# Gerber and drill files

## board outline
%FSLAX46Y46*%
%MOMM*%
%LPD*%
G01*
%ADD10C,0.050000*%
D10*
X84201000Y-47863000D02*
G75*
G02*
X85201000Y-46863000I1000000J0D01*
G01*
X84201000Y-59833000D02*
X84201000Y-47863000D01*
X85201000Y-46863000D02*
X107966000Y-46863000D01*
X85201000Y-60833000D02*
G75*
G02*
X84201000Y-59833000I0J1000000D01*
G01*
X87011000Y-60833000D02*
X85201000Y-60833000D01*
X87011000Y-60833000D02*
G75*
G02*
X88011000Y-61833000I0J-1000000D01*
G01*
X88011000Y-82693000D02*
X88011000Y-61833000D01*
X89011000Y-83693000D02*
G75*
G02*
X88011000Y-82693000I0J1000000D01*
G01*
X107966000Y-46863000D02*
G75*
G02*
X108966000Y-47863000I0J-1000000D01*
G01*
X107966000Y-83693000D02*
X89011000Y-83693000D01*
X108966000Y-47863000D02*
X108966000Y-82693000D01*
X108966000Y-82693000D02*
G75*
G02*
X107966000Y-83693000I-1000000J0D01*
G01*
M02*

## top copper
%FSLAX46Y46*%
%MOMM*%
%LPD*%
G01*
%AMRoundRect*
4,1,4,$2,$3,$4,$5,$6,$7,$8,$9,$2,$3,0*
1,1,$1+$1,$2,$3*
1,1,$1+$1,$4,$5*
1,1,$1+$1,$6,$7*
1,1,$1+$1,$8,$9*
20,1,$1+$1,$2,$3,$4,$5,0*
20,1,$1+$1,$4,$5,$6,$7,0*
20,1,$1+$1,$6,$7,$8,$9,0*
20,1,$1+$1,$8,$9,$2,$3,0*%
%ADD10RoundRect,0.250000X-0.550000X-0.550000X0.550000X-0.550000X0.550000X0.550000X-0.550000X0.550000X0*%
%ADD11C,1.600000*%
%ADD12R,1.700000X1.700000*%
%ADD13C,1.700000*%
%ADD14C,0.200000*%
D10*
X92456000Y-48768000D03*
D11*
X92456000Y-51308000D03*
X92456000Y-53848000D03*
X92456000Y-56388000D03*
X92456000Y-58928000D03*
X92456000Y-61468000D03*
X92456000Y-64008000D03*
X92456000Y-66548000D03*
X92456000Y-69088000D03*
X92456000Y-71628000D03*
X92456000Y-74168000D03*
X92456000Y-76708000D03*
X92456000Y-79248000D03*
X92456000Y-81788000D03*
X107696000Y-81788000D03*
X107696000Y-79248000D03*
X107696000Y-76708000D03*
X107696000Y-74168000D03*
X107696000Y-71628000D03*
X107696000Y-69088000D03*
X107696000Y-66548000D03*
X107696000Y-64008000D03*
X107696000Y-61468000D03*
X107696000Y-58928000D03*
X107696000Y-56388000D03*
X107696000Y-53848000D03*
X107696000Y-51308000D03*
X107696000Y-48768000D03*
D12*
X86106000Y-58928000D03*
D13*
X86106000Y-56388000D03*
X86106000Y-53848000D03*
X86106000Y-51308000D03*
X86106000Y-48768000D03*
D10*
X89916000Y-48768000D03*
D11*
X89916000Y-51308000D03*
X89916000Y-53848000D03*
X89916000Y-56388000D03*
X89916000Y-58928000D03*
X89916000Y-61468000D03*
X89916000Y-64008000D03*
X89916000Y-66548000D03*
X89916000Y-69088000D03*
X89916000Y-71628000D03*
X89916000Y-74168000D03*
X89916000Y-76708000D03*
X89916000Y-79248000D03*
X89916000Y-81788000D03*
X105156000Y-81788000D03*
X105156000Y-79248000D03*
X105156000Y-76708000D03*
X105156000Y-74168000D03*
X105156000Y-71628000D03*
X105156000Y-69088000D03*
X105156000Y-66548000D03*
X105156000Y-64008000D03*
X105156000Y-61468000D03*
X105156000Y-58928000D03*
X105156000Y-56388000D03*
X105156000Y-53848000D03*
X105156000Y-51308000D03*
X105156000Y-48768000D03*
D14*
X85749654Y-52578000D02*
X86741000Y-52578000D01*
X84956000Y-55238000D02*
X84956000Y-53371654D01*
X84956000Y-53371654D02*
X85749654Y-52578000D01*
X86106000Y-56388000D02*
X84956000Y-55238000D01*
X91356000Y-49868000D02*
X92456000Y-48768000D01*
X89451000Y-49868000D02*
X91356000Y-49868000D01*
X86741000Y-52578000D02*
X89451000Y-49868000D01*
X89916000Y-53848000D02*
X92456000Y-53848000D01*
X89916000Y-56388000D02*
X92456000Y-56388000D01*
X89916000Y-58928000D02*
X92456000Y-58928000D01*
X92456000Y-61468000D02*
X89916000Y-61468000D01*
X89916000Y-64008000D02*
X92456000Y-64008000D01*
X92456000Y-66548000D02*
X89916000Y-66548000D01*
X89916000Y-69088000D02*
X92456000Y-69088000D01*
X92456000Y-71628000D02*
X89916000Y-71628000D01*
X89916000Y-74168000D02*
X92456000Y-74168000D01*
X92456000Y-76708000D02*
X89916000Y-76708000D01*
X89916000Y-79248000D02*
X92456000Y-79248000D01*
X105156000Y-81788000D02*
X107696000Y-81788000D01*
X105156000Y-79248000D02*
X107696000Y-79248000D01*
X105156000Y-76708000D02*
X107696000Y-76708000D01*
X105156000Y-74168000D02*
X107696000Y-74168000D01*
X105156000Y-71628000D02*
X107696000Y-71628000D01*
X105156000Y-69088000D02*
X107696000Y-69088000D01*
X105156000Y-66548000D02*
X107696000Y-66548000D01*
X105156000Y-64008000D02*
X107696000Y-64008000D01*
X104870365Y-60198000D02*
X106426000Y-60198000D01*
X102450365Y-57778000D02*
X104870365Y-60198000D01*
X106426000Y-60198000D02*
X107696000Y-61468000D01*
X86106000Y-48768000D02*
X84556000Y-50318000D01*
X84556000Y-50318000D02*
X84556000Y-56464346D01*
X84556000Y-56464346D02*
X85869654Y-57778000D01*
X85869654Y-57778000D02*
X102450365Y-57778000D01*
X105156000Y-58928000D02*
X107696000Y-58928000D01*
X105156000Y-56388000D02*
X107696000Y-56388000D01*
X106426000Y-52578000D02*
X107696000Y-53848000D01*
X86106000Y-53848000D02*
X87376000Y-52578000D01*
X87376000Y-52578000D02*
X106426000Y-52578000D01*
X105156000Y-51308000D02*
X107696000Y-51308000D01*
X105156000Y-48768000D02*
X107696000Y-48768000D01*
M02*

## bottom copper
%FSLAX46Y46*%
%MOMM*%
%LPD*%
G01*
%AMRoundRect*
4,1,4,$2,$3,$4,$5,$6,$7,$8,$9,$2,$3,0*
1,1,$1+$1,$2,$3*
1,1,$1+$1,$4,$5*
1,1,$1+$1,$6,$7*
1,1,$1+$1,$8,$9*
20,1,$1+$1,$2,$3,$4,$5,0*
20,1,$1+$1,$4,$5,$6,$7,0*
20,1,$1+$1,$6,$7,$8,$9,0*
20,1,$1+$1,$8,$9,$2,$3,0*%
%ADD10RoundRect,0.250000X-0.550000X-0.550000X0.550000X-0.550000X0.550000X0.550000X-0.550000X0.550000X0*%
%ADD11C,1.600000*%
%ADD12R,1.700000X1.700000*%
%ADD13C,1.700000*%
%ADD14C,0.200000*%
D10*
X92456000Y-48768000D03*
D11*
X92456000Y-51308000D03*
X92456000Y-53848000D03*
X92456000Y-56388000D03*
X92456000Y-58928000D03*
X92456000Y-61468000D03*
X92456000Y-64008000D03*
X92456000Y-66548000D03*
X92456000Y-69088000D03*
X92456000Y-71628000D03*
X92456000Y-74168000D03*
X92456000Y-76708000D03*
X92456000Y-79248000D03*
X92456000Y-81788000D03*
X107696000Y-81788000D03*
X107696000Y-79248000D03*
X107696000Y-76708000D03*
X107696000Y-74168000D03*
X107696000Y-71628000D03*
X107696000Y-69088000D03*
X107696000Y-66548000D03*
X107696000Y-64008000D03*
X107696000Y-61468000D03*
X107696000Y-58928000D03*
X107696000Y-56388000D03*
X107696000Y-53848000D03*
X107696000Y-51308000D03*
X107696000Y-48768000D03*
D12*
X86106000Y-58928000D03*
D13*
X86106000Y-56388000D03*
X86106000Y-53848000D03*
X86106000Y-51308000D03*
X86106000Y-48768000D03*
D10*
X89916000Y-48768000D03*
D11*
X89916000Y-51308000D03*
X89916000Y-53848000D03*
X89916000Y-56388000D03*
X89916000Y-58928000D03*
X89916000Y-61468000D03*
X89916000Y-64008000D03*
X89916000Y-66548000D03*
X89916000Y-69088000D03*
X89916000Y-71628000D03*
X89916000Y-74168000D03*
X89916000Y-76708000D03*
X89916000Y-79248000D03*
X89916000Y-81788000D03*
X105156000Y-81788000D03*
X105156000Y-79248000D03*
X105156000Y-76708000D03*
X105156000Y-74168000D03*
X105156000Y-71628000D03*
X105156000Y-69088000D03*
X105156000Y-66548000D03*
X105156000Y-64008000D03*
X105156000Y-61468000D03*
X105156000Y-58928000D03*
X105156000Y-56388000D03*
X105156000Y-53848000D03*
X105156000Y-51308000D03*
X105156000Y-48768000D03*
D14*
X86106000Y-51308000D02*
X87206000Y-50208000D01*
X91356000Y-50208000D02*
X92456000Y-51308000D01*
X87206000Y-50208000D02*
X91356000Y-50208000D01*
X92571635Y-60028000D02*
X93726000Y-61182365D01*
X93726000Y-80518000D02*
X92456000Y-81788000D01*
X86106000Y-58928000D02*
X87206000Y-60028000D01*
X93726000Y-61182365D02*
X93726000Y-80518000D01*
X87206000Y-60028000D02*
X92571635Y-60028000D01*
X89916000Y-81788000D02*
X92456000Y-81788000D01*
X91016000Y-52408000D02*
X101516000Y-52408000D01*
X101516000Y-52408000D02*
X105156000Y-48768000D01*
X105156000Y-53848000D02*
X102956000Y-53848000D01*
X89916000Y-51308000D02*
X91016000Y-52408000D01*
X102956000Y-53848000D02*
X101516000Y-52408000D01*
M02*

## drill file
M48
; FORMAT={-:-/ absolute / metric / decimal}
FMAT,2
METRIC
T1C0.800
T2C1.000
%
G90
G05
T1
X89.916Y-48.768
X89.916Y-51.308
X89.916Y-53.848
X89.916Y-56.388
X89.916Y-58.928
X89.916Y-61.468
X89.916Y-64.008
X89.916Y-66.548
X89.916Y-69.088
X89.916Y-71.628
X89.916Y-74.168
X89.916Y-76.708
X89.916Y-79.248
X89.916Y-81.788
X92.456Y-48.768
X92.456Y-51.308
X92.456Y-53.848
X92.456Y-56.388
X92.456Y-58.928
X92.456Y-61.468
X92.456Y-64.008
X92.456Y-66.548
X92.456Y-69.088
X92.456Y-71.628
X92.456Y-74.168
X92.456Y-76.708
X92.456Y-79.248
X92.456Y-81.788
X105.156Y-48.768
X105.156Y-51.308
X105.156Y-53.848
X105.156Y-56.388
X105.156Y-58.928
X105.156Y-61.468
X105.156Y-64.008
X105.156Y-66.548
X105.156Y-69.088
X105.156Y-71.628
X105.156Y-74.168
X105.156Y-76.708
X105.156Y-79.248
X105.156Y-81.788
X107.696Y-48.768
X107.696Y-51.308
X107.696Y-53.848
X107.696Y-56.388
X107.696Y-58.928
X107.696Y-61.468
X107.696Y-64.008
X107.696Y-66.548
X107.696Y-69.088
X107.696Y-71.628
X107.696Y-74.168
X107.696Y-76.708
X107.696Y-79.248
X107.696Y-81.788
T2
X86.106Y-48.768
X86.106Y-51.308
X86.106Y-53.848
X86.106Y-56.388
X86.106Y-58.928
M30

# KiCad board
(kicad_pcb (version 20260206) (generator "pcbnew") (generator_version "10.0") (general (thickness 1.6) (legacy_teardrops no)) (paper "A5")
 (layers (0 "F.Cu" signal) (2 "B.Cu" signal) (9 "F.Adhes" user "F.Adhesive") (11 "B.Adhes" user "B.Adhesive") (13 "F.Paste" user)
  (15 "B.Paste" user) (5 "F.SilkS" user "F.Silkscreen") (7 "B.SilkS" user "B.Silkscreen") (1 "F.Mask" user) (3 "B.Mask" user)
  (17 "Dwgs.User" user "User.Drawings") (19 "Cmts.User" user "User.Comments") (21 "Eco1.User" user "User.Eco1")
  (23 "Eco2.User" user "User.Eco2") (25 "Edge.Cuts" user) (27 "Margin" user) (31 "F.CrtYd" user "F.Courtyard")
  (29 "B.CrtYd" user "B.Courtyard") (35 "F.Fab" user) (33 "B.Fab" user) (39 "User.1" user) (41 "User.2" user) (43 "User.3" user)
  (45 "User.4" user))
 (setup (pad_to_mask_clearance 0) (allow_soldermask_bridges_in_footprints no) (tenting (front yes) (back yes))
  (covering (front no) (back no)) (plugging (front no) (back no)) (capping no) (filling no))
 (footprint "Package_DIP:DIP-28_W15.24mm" (layer "F.Cu") (at 92.456 48.768)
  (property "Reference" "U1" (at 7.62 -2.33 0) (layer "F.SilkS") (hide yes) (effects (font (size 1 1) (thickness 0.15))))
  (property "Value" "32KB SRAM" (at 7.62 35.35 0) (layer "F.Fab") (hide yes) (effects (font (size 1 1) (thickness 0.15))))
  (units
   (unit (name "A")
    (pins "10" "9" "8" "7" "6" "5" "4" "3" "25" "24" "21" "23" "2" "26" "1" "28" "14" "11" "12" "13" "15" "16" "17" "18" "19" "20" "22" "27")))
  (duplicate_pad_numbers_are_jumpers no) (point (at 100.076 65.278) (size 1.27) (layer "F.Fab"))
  (pad "1" thru_hole roundrect (at 0 0) (size 1.6 1.6) (drill 0.8) (layers "*.Cu" "*.Mask") (remove_unused_layers no)
   (roundrect_rratio 0.15625) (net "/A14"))
  (pad "2" thru_hole circle (at 0 2.54) (size 1.6 1.6) (drill 0.8) (layers "*.Cu" "*.Mask") (remove_unused_layers no) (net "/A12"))
  (pad "3" thru_hole circle (at 0 5.08) (size 1.6 1.6) (drill 0.8) (layers "*.Cu" "*.Mask") (remove_unused_layers no) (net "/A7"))
  (pad "4" thru_hole circle (at 0 7.62) (size 1.6 1.6) (drill 0.8) (layers "*.Cu" "*.Mask") (remove_unused_layers no) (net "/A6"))
  (pad "5" thru_hole circle (at 0 10.16) (size 1.6 1.6) (drill 0.8) (layers "*.Cu" "*.Mask") (remove_unused_layers no) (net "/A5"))
  (pad "6" thru_hole circle (at 0 12.7) (size 1.6 1.6) (drill 0.8) (layers "*.Cu" "*.Mask") (remove_unused_layers no) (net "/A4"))
  (pad "7" thru_hole circle (at 0 15.24) (size 1.6 1.6) (drill 0.8) (layers "*.Cu" "*.Mask") (remove_unused_layers no) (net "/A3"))
  (pad "8" thru_hole circle (at 0 17.78) (size 1.6 1.6) (drill 0.8) (layers "*.Cu" "*.Mask") (remove_unused_layers no) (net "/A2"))
  (pad "9" thru_hole circle (at 0 20.32) (size 1.6 1.6) (drill 0.8) (layers "*.Cu" "*.Mask") (remove_unused_layers no) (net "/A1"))
  (pad "10" thru_hole circle (at 0 22.86) (size 1.6 1.6) (drill 0.8) (layers "*.Cu" "*.Mask") (remove_unused_layers no) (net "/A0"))
  (pad "11" thru_hole circle (at 0 25.4) (size 1.6 1.6) (drill 0.8) (layers "*.Cu" "*.Mask") (remove_unused_layers no) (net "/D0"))
  (pad "12" thru_hole circle (at 0 27.94) (size 1.6 1.6) (drill 0.8) (layers "*.Cu" "*.Mask") (remove_unused_layers no) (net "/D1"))
  (pad "13" thru_hole circle (at 0 30.48) (size 1.6 1.6) (drill 0.8) (layers "*.Cu" "*.Mask") (remove_unused_layers no) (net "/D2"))
  (pad "14" thru_hole circle (at 0 33.02) (size 1.6 1.6) (drill 0.8) (layers "*.Cu" "*.Mask") (remove_unused_layers no) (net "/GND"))
  (pad "15" thru_hole circle (at 15.24 33.02) (size 1.6 1.6) (drill 0.8) (layers "*.Cu" "*.Mask") (remove_unused_layers no) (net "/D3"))
  (pad "16" thru_hole circle (at 15.24 30.48) (size 1.6 1.6) (drill 0.8) (layers "*.Cu" "*.Mask") (remove_unused_layers no) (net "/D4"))
  (pad "17" thru_hole circle (at 15.24 27.94) (size 1.6 1.6) (drill 0.8) (layers "*.Cu" "*.Mask") (remove_unused_layers no) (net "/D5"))
  (pad "18" thru_hole circle (at 15.24 25.4) (size 1.6 1.6) (drill 0.8) (layers "*.Cu" "*.Mask") (remove_unused_layers no) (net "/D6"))
  (pad "19" thru_hole circle (at 15.24 22.86) (size 1.6 1.6) (drill 0.8) (layers "*.Cu" "*.Mask") (remove_unused_layers no) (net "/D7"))
  (pad "20" thru_hole circle (at 15.24 20.32) (size 1.6 1.6) (drill 0.8) (layers "*.Cu" "*.Mask") (remove_unused_layers no) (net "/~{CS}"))
  (pad "21" thru_hole circle (at 15.24 17.78) (size 1.6 1.6) (drill 0.8) (layers "*.Cu" "*.Mask") (remove_unused_layers no) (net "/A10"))
  (pad "22" thru_hole circle (at 15.24 15.24) (size 1.6 1.6) (drill 0.8) (layers "*.Cu" "*.Mask") (remove_unused_layers no) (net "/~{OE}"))
  (pad "23" thru_hole circle (at 15.24 12.7) (size 1.6 1.6) (drill 0.8) (layers "*.Cu" "*.Mask") (remove_unused_layers no) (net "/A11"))
  (pad "24" thru_hole circle (at 15.24 10.16) (size 1.6 1.6) (drill 0.8) (layers "*.Cu" "*.Mask") (remove_unused_layers no) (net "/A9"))
  (pad "25" thru_hole circle (at 15.24 7.62) (size 1.6 1.6) (drill 0.8) (layers "*.Cu" "*.Mask") (remove_unused_layers no) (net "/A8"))
  (pad "26" thru_hole circle (at 15.24 5.08) (size 1.6 1.6) (drill 0.8) (layers "*.Cu" "*.Mask") (remove_unused_layers no) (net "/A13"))
  (pad "27" thru_hole circle (at 15.24 2.54) (size 1.6 1.6) (drill 0.8) (layers "*.Cu" "*.Mask") (remove_unused_layers no) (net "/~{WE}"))
  (pad "28" thru_hole circle (at 15.24 0) (size 1.6 1.6) (drill 0.8) (layers "*.Cu" "*.Mask") (remove_unused_layers no) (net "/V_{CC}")))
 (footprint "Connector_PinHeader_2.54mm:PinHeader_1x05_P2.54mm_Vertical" (layer "F.Cu") (at 86.106 58.928 180)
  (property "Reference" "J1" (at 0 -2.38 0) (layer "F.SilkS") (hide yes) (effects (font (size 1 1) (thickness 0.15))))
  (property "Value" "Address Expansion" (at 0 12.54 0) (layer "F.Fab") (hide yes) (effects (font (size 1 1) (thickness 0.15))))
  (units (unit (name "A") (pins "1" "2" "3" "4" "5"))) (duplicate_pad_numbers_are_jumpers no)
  (pad "1" thru_hole rect (at 0 0 180) (size 1.7 1.7) (drill 1) (layers "*.Cu" "*.Mask") (remove_unused_layers no) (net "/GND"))
  (pad "2" thru_hole circle (at 0 2.54 180) (size 1.7 1.7) (drill 1) (layers "*.Cu" "*.Mask") (remove_unused_layers no) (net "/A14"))
  (pad "3" thru_hole circle (at 0 5.08 180) (size 1.7 1.7) (drill 1) (layers "*.Cu" "*.Mask") (remove_unused_layers no) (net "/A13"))
  (pad "4" thru_hole circle (at 0 7.62 180) (size 1.7 1.7) (drill 1) (layers "*.Cu" "*.Mask") (remove_unused_layers no) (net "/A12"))
  (pad "5" thru_hole circle (at 0 10.16 180) (size 1.7 1.7) (drill 1) (layers "*.Cu" "*.Mask") (remove_unused_layers no) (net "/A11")))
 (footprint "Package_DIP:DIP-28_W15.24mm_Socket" (layer "F.Cu") (at 89.916 48.768)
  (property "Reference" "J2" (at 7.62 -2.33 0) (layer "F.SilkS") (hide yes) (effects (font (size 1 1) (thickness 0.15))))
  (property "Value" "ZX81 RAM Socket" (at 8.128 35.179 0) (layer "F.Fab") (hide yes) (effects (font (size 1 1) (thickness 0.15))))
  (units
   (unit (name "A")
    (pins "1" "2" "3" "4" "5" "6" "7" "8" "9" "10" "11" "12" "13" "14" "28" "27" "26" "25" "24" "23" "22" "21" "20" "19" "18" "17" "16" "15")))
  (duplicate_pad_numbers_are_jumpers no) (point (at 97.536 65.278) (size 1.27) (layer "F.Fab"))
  (pad "1" thru_hole roundrect (at 0 0) (size 1.6 1.6) (drill 0.8) (layers "*.Cu" "*.Mask") (remove_unused_layers no)
   (roundrect_rratio 0.15625) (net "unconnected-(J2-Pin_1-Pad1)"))
  (pad "2" thru_hole circle (at 0 2.54) (size 1.6 1.6) (drill 0.8) (layers "*.Cu" "*.Mask") (remove_unused_layers no) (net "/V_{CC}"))
  (pad "3" thru_hole circle (at 0 5.08) (size 1.6 1.6) (drill 0.8) (layers "*.Cu" "*.Mask") (remove_unused_layers no) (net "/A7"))
  (pad "4" thru_hole circle (at 0 7.62) (size 1.6 1.6) (drill 0.8) (layers "*.Cu" "*.Mask") (remove_unused_layers no) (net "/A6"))
  (pad "5" thru_hole circle (at 0 10.16) (size 1.6 1.6) (drill 0.8) (layers "*.Cu" "*.Mask") (remove_unused_layers no) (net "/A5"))
  (pad "6" thru_hole circle (at 0 12.7) (size 1.6 1.6) (drill 0.8) (layers "*.Cu" "*.Mask") (remove_unused_layers no) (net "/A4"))
  (pad "7" thru_hole circle (at 0 15.24) (size 1.6 1.6) (drill 0.8) (layers "*.Cu" "*.Mask") (remove_unused_layers no) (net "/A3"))
  (pad "8" thru_hole circle (at 0 17.78) (size 1.6 1.6) (drill 0.8) (layers "*.Cu" "*.Mask") (remove_unused_layers no) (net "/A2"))
  (pad "9" thru_hole circle (at 0 20.32) (size 1.6 1.6) (drill 0.8) (layers "*.Cu" "*.Mask") (remove_unused_layers no) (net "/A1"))
  (pad "10" thru_hole circle (at 0 22.86) (size 1.6 1.6) (drill 0.8) (layers "*.Cu" "*.Mask") (remove_unused_layers no) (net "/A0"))
  (pad "11" thru_hole circle (at 0 25.4) (size 1.6 1.6) (drill 0.8) (layers "*.Cu" "*.Mask") (remove_unused_layers no) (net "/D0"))
  (pad "12" thru_hole circle (at 0 27.94) (size 1.6 1.6) (drill 0.8) (layers "*.Cu" "*.Mask") (remove_unused_layers no) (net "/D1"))
  (pad "13" thru_hole circle (at 0 30.48) (size 1.6 1.6) (drill 0.8) (layers "*.Cu" "*.Mask") (remove_unused_layers no) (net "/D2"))
  (pad "14" thru_hole circle (at 0 33.02) (size 1.6 1.6) (drill 0.8) (layers "*.Cu" "*.Mask") (remove_unused_layers no) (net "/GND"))
  (pad "15" thru_hole circle (at 15.24 33.02) (size 1.6 1.6) (drill 0.8) (layers "*.Cu" "*.Mask") (remove_unused_layers no) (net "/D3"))
  (pad "16" thru_hole circle (at 15.24 30.48) (size 1.6 1.6) (drill 0.8) (layers "*.Cu" "*.Mask") (remove_unused_layers no) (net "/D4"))
  (pad "17" thru_hole circle (at 15.24 27.94) (size 1.6 1.6) (drill 0.8) (layers "*.Cu" "*.Mask") (remove_unused_layers no) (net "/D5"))
  (pad "18" thru_hole circle (at 15.24 25.4) (size 1.6 1.6) (drill 0.8) (layers "*.Cu" "*.Mask") (remove_unused_layers no) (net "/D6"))
  (pad "19" thru_hole circle (at 15.24 22.86) (size 1.6 1.6) (drill 0.8) (layers "*.Cu" "*.Mask") (remove_unused_layers no) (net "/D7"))
  (pad "20" thru_hole circle (at 15.24 20.32) (size 1.6 1.6) (drill 0.8) (layers "*.Cu" "*.Mask") (remove_unused_layers no) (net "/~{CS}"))
  (pad "21" thru_hole circle (at 15.24 17.78) (size 1.6 1.6) (drill 0.8) (layers "*.Cu" "*.Mask") (remove_unused_layers no) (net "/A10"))
  (pad "22" thru_hole circle (at 15.24 15.24) (size 1.6 1.6) (drill 0.8) (layers "*.Cu" "*.Mask") (remove_unused_layers no) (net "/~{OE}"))
  (pad "23" thru_hole circle (at 15.24 12.7) (size 1.6 1.6) (drill 0.8) (layers "*.Cu" "*.Mask") (remove_unused_layers no)
   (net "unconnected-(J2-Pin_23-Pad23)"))
  (pad "24" thru_hole circle (at 15.24 10.16) (size 1.6 1.6) (drill 0.8) (layers "*.Cu" "*.Mask") (remove_unused_layers no) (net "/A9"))
  (pad "25" thru_hole circle (at 15.24 7.62) (size 1.6 1.6) (drill 0.8) (layers "*.Cu" "*.Mask") (remove_unused_layers no) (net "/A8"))
  (pad "26" thru_hole circle (at 15.24 5.08) (size 1.6 1.6) (drill 0.8) (layers "*.Cu" "*.Mask") (remove_unused_layers no) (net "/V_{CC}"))
  (pad "27" thru_hole circle (at 15.24 2.54) (size 1.6 1.6) (drill 0.8) (layers "*.Cu" "*.Mask") (remove_unused_layers no) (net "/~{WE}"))
  (pad "28" thru_hole circle (at 15.24 0) (size 1.6 1.6) (drill 0.8) (layers "*.Cu" "*.Mask") (remove_unused_layers no) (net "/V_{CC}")))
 (gr_arc (start 84.201 47.863) (mid 84.493893 47.155893) (end 85.201 46.863) (stroke (width 0.05) (type default)) (layer "Edge.Cuts"))
 (gr_line (start 84.201 59.833) (end 84.201 47.863) (stroke (width 0.05) (type default)) (layer "Edge.Cuts"))
 (gr_line (start 85.201 46.863) (end 107.966 46.863) (stroke (width 0.05) (type default)) (layer "Edge.Cuts"))
 (gr_arc (start 85.201 60.833) (mid 84.493893 60.540107) (end 84.201 59.833) (stroke (width 0.05) (type default)) (layer "Edge.Cuts"))
 (gr_line (start 87.011 60.833) (end 85.201 60.833) (stroke (width 0.05) (type default)) (layer "Edge.Cuts"))
 (gr_arc (start 87.011 60.833) (mid 87.718107 61.125893) (end 88.011 61.833) (stroke (width 0.05) (type default)) (layer "Edge.Cuts"))
 (gr_line (start 88.011 82.693) (end 88.011 61.833) (stroke (width 0.05) (type default)) (layer "Edge.Cuts"))
 (gr_arc (start 89.011 83.693) (mid 88.303893 83.400107) (end 88.011 82.693) (stroke (width 0.05) (type default)) (layer "Edge.Cuts"))
 (gr_arc (start 107.966 46.863) (mid 108.673107 47.155893) (end 108.966 47.863) (stroke (width 0.05) (type default)) (layer "Edge.Cuts"))
 (gr_line (start 107.966 83.693) (end 89.011 83.693) (stroke (width 0.05) (type default)) (layer "Edge.Cuts"))
 (gr_line (start 108.966 47.863) (end 108.966 82.693) (stroke (width 0.05) (type default)) (layer "Edge.Cuts"))
 (gr_arc (start 108.966 82.693) (mid 108.673107 83.400107) (end 107.966 83.693) (stroke (width 0.05) (type default)) (layer "Edge.Cuts"))
 (segment (start 85.749654 52.578) (end 86.741 52.578) (width 0.2) (layer "F.Cu") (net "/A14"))
 (segment (start 84.956 55.238) (end 84.956 53.371654) (width 0.2) (layer "F.Cu") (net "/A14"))
 (segment (start 84.956 53.371654) (end 85.749654 52.578) (width 0.2) (layer "F.Cu") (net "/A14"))
 (segment (start 86.106 56.388) (end 84.956 55.238) (width 0.2) (layer "F.Cu") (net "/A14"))
 (segment (start 91.356 49.868) (end 92.456 48.768) (width 0.2) (layer "F.Cu") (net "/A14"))
 (segment (start 89.451 49.868) (end 91.356 49.868) (width 0.2) (layer "F.Cu") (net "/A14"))
 (segment (start 86.741 52.578) (end 89.451 49.868) (width 0.2) (layer "F.Cu") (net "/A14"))
 (segment (start 86.106 51.308) (end 87.206 50.208) (width 0.2) (layer "B.Cu") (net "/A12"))
 (segment (start 91.356 50.208) (end 92.456 51.308) (width 0.2) (layer "B.Cu") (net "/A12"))
 (segment (start 87.206 50.208) (end 91.356 50.208) (width 0.2) (layer "B.Cu") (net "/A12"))
 (segment (start 89.916 53.848) (end 92.456 53.848) (width 0.2) (layer "F.Cu") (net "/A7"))
 (segment (start 89.916 56.388) (end 92.456 56.388) (width 0.2) (layer "F.Cu") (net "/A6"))
 (segment (start 89.916 58.928) (end 92.456 58.928) (width 0.2) (layer "F.Cu") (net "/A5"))
 (segment (start 92.456 61.468) (end 89.916 61.468) (width 0.2) (layer "F.Cu") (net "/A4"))
 (segment (start 89.916 64.008) (end 92.456 64.008) (width 0.2) (layer "F.Cu") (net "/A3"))
 (segment (start 92.456 66.548) (end 89.916 66.548) (width 0.2) (layer "F.Cu") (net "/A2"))
 (segment (start 89.916 69.088) (end 92.456 69.088) (width 0.2) (layer "F.Cu") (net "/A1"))
 (segment (start 92.456 71.628) (end 89.916 71.628) (width 0.2) (layer "F.Cu") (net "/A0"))
 (segment (start 89.916 74.168) (end 92.456 74.168) (width 0.2) (layer "F.Cu") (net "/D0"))
 (segment (start 92.456 76.708) (end 89.916 76.708) (width 0.2) (layer "F.Cu") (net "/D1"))
 (segment (start 89.916 79.248) (end 92.456 79.248) (width 0.2) (layer "F.Cu") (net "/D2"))
 (segment (start 92.571635 60.028) (end 93.726 61.182365) (width 0.2) (layer "B.Cu") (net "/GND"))
 (segment (start 93.726 80.518) (end 92.456 81.788) (width 0.2) (layer "B.Cu") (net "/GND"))
 (segment (start 86.106 58.928) (end 87.206 60.028) (width 0.2) (layer "B.Cu") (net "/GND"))
 (segment (start 93.726 61.182365) (end 93.726 80.518) (width 0.2) (layer "B.Cu") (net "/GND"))
 (segment (start 87.206 60.028) (end 92.571635 60.028) (width 0.2) (layer "B.Cu") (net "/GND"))
 (segment (start 89.916 81.788) (end 92.456 81.788) (width 0.2) (layer "B.Cu") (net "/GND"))
 (segment (start 105.156 81.788) (end 107.696 81.788) (width 0.2) (layer "F.Cu") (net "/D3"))
 (segment (start 105.156 79.248) (end 107.696 79.248) (width 0.2) (layer "F.Cu") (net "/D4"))
 (segment (start 105.156 76.708) (end 107.696 76.708) (width 0.2) (layer "F.Cu") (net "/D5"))
 (segment (start 105.156 74.168) (end 107.696 74.168) (width 0.2) (layer "F.Cu") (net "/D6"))
 (segment (start 105.156 71.628) (end 107.696 71.628) (width 0.2) (layer "F.Cu") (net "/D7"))
 (segment (start 105.156 69.088) (end 107.696 69.088) (width 0.2) (layer "F.Cu") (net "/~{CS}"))
 (segment (start 105.156 66.548) (end 107.696 66.548) (width 0.2) (layer "F.Cu") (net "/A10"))
 (segment (start 105.156 64.008) (end 107.696 64.008) (width 0.2) (layer "F.Cu") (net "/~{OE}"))
 (segment (start 104.870365 60.198) (end 106.426 60.198) (width 0.2) (layer "F.Cu") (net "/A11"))
 (segment (start 102.450365 57.778) (end 104.870365 60.198) (width 0.2) (layer "F.Cu") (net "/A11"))
 (segment (start 106.426 60.198) (end 107.696 61.468) (width 0.2) (layer "F.Cu") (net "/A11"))
 (segment (start 86.106 48.768) (end 84.556 50.318) (width 0.2) (layer "F.Cu") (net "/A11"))
 (segment (start 84.556 50.318) (end 84.556 56.464346) (width 0.2) (layer "F.Cu") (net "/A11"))
 (segment (start 84.556 56.464346) (end 85.869654 57.778) (width 0.2) (layer "F.Cu") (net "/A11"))
 (segment (start 85.869654 57.778) (end 102.450365 57.778) (width 0.2) (layer "F.Cu") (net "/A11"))
 (segment (start 105.156 58.928) (end 107.696 58.928) (width 0.2) (layer "F.Cu") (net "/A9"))
 (segment (start 105.156 56.388) (end 107.696 56.388) (width 0.2) (layer "F.Cu") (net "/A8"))
 (segment (start 106.426 52.578) (end 107.696 53.848) (width 0.2) (layer "F.Cu") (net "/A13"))
 (segment (start 86.106 53.848) (end 87.376 52.578) (width 0.2) (layer "F.Cu") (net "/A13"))
 (segment (start 87.376 52.578) (end 106.426 52.578) (width 0.2) (layer "F.Cu") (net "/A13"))
 (segment (start 105.156 51.308) (end 107.696 51.308) (width 0.2) (layer "F.Cu") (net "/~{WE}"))
 (segment (start 105.156 48.768) (end 107.696 48.768) (width 0.2) (layer "F.Cu") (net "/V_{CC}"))
 (segment (start 91.016 52.408) (end 101.516 52.408) (width 0.2) (layer "B.Cu") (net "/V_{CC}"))
 (segment (start 101.516 52.408) (end 105.156 48.768) (width 0.2) (layer "B.Cu") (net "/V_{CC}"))
 (segment (start 105.156 53.848) (end 102.956 53.848) (width 0.2) (layer "B.Cu") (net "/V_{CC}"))
 (segment (start 89.916 51.308) (end 91.016 52.408) (width 0.2) (layer "B.Cu") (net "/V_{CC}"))
 (segment (start 102.956 53.848) (end 101.516 52.408) (width 0.2) (layer "B.Cu") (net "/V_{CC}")))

